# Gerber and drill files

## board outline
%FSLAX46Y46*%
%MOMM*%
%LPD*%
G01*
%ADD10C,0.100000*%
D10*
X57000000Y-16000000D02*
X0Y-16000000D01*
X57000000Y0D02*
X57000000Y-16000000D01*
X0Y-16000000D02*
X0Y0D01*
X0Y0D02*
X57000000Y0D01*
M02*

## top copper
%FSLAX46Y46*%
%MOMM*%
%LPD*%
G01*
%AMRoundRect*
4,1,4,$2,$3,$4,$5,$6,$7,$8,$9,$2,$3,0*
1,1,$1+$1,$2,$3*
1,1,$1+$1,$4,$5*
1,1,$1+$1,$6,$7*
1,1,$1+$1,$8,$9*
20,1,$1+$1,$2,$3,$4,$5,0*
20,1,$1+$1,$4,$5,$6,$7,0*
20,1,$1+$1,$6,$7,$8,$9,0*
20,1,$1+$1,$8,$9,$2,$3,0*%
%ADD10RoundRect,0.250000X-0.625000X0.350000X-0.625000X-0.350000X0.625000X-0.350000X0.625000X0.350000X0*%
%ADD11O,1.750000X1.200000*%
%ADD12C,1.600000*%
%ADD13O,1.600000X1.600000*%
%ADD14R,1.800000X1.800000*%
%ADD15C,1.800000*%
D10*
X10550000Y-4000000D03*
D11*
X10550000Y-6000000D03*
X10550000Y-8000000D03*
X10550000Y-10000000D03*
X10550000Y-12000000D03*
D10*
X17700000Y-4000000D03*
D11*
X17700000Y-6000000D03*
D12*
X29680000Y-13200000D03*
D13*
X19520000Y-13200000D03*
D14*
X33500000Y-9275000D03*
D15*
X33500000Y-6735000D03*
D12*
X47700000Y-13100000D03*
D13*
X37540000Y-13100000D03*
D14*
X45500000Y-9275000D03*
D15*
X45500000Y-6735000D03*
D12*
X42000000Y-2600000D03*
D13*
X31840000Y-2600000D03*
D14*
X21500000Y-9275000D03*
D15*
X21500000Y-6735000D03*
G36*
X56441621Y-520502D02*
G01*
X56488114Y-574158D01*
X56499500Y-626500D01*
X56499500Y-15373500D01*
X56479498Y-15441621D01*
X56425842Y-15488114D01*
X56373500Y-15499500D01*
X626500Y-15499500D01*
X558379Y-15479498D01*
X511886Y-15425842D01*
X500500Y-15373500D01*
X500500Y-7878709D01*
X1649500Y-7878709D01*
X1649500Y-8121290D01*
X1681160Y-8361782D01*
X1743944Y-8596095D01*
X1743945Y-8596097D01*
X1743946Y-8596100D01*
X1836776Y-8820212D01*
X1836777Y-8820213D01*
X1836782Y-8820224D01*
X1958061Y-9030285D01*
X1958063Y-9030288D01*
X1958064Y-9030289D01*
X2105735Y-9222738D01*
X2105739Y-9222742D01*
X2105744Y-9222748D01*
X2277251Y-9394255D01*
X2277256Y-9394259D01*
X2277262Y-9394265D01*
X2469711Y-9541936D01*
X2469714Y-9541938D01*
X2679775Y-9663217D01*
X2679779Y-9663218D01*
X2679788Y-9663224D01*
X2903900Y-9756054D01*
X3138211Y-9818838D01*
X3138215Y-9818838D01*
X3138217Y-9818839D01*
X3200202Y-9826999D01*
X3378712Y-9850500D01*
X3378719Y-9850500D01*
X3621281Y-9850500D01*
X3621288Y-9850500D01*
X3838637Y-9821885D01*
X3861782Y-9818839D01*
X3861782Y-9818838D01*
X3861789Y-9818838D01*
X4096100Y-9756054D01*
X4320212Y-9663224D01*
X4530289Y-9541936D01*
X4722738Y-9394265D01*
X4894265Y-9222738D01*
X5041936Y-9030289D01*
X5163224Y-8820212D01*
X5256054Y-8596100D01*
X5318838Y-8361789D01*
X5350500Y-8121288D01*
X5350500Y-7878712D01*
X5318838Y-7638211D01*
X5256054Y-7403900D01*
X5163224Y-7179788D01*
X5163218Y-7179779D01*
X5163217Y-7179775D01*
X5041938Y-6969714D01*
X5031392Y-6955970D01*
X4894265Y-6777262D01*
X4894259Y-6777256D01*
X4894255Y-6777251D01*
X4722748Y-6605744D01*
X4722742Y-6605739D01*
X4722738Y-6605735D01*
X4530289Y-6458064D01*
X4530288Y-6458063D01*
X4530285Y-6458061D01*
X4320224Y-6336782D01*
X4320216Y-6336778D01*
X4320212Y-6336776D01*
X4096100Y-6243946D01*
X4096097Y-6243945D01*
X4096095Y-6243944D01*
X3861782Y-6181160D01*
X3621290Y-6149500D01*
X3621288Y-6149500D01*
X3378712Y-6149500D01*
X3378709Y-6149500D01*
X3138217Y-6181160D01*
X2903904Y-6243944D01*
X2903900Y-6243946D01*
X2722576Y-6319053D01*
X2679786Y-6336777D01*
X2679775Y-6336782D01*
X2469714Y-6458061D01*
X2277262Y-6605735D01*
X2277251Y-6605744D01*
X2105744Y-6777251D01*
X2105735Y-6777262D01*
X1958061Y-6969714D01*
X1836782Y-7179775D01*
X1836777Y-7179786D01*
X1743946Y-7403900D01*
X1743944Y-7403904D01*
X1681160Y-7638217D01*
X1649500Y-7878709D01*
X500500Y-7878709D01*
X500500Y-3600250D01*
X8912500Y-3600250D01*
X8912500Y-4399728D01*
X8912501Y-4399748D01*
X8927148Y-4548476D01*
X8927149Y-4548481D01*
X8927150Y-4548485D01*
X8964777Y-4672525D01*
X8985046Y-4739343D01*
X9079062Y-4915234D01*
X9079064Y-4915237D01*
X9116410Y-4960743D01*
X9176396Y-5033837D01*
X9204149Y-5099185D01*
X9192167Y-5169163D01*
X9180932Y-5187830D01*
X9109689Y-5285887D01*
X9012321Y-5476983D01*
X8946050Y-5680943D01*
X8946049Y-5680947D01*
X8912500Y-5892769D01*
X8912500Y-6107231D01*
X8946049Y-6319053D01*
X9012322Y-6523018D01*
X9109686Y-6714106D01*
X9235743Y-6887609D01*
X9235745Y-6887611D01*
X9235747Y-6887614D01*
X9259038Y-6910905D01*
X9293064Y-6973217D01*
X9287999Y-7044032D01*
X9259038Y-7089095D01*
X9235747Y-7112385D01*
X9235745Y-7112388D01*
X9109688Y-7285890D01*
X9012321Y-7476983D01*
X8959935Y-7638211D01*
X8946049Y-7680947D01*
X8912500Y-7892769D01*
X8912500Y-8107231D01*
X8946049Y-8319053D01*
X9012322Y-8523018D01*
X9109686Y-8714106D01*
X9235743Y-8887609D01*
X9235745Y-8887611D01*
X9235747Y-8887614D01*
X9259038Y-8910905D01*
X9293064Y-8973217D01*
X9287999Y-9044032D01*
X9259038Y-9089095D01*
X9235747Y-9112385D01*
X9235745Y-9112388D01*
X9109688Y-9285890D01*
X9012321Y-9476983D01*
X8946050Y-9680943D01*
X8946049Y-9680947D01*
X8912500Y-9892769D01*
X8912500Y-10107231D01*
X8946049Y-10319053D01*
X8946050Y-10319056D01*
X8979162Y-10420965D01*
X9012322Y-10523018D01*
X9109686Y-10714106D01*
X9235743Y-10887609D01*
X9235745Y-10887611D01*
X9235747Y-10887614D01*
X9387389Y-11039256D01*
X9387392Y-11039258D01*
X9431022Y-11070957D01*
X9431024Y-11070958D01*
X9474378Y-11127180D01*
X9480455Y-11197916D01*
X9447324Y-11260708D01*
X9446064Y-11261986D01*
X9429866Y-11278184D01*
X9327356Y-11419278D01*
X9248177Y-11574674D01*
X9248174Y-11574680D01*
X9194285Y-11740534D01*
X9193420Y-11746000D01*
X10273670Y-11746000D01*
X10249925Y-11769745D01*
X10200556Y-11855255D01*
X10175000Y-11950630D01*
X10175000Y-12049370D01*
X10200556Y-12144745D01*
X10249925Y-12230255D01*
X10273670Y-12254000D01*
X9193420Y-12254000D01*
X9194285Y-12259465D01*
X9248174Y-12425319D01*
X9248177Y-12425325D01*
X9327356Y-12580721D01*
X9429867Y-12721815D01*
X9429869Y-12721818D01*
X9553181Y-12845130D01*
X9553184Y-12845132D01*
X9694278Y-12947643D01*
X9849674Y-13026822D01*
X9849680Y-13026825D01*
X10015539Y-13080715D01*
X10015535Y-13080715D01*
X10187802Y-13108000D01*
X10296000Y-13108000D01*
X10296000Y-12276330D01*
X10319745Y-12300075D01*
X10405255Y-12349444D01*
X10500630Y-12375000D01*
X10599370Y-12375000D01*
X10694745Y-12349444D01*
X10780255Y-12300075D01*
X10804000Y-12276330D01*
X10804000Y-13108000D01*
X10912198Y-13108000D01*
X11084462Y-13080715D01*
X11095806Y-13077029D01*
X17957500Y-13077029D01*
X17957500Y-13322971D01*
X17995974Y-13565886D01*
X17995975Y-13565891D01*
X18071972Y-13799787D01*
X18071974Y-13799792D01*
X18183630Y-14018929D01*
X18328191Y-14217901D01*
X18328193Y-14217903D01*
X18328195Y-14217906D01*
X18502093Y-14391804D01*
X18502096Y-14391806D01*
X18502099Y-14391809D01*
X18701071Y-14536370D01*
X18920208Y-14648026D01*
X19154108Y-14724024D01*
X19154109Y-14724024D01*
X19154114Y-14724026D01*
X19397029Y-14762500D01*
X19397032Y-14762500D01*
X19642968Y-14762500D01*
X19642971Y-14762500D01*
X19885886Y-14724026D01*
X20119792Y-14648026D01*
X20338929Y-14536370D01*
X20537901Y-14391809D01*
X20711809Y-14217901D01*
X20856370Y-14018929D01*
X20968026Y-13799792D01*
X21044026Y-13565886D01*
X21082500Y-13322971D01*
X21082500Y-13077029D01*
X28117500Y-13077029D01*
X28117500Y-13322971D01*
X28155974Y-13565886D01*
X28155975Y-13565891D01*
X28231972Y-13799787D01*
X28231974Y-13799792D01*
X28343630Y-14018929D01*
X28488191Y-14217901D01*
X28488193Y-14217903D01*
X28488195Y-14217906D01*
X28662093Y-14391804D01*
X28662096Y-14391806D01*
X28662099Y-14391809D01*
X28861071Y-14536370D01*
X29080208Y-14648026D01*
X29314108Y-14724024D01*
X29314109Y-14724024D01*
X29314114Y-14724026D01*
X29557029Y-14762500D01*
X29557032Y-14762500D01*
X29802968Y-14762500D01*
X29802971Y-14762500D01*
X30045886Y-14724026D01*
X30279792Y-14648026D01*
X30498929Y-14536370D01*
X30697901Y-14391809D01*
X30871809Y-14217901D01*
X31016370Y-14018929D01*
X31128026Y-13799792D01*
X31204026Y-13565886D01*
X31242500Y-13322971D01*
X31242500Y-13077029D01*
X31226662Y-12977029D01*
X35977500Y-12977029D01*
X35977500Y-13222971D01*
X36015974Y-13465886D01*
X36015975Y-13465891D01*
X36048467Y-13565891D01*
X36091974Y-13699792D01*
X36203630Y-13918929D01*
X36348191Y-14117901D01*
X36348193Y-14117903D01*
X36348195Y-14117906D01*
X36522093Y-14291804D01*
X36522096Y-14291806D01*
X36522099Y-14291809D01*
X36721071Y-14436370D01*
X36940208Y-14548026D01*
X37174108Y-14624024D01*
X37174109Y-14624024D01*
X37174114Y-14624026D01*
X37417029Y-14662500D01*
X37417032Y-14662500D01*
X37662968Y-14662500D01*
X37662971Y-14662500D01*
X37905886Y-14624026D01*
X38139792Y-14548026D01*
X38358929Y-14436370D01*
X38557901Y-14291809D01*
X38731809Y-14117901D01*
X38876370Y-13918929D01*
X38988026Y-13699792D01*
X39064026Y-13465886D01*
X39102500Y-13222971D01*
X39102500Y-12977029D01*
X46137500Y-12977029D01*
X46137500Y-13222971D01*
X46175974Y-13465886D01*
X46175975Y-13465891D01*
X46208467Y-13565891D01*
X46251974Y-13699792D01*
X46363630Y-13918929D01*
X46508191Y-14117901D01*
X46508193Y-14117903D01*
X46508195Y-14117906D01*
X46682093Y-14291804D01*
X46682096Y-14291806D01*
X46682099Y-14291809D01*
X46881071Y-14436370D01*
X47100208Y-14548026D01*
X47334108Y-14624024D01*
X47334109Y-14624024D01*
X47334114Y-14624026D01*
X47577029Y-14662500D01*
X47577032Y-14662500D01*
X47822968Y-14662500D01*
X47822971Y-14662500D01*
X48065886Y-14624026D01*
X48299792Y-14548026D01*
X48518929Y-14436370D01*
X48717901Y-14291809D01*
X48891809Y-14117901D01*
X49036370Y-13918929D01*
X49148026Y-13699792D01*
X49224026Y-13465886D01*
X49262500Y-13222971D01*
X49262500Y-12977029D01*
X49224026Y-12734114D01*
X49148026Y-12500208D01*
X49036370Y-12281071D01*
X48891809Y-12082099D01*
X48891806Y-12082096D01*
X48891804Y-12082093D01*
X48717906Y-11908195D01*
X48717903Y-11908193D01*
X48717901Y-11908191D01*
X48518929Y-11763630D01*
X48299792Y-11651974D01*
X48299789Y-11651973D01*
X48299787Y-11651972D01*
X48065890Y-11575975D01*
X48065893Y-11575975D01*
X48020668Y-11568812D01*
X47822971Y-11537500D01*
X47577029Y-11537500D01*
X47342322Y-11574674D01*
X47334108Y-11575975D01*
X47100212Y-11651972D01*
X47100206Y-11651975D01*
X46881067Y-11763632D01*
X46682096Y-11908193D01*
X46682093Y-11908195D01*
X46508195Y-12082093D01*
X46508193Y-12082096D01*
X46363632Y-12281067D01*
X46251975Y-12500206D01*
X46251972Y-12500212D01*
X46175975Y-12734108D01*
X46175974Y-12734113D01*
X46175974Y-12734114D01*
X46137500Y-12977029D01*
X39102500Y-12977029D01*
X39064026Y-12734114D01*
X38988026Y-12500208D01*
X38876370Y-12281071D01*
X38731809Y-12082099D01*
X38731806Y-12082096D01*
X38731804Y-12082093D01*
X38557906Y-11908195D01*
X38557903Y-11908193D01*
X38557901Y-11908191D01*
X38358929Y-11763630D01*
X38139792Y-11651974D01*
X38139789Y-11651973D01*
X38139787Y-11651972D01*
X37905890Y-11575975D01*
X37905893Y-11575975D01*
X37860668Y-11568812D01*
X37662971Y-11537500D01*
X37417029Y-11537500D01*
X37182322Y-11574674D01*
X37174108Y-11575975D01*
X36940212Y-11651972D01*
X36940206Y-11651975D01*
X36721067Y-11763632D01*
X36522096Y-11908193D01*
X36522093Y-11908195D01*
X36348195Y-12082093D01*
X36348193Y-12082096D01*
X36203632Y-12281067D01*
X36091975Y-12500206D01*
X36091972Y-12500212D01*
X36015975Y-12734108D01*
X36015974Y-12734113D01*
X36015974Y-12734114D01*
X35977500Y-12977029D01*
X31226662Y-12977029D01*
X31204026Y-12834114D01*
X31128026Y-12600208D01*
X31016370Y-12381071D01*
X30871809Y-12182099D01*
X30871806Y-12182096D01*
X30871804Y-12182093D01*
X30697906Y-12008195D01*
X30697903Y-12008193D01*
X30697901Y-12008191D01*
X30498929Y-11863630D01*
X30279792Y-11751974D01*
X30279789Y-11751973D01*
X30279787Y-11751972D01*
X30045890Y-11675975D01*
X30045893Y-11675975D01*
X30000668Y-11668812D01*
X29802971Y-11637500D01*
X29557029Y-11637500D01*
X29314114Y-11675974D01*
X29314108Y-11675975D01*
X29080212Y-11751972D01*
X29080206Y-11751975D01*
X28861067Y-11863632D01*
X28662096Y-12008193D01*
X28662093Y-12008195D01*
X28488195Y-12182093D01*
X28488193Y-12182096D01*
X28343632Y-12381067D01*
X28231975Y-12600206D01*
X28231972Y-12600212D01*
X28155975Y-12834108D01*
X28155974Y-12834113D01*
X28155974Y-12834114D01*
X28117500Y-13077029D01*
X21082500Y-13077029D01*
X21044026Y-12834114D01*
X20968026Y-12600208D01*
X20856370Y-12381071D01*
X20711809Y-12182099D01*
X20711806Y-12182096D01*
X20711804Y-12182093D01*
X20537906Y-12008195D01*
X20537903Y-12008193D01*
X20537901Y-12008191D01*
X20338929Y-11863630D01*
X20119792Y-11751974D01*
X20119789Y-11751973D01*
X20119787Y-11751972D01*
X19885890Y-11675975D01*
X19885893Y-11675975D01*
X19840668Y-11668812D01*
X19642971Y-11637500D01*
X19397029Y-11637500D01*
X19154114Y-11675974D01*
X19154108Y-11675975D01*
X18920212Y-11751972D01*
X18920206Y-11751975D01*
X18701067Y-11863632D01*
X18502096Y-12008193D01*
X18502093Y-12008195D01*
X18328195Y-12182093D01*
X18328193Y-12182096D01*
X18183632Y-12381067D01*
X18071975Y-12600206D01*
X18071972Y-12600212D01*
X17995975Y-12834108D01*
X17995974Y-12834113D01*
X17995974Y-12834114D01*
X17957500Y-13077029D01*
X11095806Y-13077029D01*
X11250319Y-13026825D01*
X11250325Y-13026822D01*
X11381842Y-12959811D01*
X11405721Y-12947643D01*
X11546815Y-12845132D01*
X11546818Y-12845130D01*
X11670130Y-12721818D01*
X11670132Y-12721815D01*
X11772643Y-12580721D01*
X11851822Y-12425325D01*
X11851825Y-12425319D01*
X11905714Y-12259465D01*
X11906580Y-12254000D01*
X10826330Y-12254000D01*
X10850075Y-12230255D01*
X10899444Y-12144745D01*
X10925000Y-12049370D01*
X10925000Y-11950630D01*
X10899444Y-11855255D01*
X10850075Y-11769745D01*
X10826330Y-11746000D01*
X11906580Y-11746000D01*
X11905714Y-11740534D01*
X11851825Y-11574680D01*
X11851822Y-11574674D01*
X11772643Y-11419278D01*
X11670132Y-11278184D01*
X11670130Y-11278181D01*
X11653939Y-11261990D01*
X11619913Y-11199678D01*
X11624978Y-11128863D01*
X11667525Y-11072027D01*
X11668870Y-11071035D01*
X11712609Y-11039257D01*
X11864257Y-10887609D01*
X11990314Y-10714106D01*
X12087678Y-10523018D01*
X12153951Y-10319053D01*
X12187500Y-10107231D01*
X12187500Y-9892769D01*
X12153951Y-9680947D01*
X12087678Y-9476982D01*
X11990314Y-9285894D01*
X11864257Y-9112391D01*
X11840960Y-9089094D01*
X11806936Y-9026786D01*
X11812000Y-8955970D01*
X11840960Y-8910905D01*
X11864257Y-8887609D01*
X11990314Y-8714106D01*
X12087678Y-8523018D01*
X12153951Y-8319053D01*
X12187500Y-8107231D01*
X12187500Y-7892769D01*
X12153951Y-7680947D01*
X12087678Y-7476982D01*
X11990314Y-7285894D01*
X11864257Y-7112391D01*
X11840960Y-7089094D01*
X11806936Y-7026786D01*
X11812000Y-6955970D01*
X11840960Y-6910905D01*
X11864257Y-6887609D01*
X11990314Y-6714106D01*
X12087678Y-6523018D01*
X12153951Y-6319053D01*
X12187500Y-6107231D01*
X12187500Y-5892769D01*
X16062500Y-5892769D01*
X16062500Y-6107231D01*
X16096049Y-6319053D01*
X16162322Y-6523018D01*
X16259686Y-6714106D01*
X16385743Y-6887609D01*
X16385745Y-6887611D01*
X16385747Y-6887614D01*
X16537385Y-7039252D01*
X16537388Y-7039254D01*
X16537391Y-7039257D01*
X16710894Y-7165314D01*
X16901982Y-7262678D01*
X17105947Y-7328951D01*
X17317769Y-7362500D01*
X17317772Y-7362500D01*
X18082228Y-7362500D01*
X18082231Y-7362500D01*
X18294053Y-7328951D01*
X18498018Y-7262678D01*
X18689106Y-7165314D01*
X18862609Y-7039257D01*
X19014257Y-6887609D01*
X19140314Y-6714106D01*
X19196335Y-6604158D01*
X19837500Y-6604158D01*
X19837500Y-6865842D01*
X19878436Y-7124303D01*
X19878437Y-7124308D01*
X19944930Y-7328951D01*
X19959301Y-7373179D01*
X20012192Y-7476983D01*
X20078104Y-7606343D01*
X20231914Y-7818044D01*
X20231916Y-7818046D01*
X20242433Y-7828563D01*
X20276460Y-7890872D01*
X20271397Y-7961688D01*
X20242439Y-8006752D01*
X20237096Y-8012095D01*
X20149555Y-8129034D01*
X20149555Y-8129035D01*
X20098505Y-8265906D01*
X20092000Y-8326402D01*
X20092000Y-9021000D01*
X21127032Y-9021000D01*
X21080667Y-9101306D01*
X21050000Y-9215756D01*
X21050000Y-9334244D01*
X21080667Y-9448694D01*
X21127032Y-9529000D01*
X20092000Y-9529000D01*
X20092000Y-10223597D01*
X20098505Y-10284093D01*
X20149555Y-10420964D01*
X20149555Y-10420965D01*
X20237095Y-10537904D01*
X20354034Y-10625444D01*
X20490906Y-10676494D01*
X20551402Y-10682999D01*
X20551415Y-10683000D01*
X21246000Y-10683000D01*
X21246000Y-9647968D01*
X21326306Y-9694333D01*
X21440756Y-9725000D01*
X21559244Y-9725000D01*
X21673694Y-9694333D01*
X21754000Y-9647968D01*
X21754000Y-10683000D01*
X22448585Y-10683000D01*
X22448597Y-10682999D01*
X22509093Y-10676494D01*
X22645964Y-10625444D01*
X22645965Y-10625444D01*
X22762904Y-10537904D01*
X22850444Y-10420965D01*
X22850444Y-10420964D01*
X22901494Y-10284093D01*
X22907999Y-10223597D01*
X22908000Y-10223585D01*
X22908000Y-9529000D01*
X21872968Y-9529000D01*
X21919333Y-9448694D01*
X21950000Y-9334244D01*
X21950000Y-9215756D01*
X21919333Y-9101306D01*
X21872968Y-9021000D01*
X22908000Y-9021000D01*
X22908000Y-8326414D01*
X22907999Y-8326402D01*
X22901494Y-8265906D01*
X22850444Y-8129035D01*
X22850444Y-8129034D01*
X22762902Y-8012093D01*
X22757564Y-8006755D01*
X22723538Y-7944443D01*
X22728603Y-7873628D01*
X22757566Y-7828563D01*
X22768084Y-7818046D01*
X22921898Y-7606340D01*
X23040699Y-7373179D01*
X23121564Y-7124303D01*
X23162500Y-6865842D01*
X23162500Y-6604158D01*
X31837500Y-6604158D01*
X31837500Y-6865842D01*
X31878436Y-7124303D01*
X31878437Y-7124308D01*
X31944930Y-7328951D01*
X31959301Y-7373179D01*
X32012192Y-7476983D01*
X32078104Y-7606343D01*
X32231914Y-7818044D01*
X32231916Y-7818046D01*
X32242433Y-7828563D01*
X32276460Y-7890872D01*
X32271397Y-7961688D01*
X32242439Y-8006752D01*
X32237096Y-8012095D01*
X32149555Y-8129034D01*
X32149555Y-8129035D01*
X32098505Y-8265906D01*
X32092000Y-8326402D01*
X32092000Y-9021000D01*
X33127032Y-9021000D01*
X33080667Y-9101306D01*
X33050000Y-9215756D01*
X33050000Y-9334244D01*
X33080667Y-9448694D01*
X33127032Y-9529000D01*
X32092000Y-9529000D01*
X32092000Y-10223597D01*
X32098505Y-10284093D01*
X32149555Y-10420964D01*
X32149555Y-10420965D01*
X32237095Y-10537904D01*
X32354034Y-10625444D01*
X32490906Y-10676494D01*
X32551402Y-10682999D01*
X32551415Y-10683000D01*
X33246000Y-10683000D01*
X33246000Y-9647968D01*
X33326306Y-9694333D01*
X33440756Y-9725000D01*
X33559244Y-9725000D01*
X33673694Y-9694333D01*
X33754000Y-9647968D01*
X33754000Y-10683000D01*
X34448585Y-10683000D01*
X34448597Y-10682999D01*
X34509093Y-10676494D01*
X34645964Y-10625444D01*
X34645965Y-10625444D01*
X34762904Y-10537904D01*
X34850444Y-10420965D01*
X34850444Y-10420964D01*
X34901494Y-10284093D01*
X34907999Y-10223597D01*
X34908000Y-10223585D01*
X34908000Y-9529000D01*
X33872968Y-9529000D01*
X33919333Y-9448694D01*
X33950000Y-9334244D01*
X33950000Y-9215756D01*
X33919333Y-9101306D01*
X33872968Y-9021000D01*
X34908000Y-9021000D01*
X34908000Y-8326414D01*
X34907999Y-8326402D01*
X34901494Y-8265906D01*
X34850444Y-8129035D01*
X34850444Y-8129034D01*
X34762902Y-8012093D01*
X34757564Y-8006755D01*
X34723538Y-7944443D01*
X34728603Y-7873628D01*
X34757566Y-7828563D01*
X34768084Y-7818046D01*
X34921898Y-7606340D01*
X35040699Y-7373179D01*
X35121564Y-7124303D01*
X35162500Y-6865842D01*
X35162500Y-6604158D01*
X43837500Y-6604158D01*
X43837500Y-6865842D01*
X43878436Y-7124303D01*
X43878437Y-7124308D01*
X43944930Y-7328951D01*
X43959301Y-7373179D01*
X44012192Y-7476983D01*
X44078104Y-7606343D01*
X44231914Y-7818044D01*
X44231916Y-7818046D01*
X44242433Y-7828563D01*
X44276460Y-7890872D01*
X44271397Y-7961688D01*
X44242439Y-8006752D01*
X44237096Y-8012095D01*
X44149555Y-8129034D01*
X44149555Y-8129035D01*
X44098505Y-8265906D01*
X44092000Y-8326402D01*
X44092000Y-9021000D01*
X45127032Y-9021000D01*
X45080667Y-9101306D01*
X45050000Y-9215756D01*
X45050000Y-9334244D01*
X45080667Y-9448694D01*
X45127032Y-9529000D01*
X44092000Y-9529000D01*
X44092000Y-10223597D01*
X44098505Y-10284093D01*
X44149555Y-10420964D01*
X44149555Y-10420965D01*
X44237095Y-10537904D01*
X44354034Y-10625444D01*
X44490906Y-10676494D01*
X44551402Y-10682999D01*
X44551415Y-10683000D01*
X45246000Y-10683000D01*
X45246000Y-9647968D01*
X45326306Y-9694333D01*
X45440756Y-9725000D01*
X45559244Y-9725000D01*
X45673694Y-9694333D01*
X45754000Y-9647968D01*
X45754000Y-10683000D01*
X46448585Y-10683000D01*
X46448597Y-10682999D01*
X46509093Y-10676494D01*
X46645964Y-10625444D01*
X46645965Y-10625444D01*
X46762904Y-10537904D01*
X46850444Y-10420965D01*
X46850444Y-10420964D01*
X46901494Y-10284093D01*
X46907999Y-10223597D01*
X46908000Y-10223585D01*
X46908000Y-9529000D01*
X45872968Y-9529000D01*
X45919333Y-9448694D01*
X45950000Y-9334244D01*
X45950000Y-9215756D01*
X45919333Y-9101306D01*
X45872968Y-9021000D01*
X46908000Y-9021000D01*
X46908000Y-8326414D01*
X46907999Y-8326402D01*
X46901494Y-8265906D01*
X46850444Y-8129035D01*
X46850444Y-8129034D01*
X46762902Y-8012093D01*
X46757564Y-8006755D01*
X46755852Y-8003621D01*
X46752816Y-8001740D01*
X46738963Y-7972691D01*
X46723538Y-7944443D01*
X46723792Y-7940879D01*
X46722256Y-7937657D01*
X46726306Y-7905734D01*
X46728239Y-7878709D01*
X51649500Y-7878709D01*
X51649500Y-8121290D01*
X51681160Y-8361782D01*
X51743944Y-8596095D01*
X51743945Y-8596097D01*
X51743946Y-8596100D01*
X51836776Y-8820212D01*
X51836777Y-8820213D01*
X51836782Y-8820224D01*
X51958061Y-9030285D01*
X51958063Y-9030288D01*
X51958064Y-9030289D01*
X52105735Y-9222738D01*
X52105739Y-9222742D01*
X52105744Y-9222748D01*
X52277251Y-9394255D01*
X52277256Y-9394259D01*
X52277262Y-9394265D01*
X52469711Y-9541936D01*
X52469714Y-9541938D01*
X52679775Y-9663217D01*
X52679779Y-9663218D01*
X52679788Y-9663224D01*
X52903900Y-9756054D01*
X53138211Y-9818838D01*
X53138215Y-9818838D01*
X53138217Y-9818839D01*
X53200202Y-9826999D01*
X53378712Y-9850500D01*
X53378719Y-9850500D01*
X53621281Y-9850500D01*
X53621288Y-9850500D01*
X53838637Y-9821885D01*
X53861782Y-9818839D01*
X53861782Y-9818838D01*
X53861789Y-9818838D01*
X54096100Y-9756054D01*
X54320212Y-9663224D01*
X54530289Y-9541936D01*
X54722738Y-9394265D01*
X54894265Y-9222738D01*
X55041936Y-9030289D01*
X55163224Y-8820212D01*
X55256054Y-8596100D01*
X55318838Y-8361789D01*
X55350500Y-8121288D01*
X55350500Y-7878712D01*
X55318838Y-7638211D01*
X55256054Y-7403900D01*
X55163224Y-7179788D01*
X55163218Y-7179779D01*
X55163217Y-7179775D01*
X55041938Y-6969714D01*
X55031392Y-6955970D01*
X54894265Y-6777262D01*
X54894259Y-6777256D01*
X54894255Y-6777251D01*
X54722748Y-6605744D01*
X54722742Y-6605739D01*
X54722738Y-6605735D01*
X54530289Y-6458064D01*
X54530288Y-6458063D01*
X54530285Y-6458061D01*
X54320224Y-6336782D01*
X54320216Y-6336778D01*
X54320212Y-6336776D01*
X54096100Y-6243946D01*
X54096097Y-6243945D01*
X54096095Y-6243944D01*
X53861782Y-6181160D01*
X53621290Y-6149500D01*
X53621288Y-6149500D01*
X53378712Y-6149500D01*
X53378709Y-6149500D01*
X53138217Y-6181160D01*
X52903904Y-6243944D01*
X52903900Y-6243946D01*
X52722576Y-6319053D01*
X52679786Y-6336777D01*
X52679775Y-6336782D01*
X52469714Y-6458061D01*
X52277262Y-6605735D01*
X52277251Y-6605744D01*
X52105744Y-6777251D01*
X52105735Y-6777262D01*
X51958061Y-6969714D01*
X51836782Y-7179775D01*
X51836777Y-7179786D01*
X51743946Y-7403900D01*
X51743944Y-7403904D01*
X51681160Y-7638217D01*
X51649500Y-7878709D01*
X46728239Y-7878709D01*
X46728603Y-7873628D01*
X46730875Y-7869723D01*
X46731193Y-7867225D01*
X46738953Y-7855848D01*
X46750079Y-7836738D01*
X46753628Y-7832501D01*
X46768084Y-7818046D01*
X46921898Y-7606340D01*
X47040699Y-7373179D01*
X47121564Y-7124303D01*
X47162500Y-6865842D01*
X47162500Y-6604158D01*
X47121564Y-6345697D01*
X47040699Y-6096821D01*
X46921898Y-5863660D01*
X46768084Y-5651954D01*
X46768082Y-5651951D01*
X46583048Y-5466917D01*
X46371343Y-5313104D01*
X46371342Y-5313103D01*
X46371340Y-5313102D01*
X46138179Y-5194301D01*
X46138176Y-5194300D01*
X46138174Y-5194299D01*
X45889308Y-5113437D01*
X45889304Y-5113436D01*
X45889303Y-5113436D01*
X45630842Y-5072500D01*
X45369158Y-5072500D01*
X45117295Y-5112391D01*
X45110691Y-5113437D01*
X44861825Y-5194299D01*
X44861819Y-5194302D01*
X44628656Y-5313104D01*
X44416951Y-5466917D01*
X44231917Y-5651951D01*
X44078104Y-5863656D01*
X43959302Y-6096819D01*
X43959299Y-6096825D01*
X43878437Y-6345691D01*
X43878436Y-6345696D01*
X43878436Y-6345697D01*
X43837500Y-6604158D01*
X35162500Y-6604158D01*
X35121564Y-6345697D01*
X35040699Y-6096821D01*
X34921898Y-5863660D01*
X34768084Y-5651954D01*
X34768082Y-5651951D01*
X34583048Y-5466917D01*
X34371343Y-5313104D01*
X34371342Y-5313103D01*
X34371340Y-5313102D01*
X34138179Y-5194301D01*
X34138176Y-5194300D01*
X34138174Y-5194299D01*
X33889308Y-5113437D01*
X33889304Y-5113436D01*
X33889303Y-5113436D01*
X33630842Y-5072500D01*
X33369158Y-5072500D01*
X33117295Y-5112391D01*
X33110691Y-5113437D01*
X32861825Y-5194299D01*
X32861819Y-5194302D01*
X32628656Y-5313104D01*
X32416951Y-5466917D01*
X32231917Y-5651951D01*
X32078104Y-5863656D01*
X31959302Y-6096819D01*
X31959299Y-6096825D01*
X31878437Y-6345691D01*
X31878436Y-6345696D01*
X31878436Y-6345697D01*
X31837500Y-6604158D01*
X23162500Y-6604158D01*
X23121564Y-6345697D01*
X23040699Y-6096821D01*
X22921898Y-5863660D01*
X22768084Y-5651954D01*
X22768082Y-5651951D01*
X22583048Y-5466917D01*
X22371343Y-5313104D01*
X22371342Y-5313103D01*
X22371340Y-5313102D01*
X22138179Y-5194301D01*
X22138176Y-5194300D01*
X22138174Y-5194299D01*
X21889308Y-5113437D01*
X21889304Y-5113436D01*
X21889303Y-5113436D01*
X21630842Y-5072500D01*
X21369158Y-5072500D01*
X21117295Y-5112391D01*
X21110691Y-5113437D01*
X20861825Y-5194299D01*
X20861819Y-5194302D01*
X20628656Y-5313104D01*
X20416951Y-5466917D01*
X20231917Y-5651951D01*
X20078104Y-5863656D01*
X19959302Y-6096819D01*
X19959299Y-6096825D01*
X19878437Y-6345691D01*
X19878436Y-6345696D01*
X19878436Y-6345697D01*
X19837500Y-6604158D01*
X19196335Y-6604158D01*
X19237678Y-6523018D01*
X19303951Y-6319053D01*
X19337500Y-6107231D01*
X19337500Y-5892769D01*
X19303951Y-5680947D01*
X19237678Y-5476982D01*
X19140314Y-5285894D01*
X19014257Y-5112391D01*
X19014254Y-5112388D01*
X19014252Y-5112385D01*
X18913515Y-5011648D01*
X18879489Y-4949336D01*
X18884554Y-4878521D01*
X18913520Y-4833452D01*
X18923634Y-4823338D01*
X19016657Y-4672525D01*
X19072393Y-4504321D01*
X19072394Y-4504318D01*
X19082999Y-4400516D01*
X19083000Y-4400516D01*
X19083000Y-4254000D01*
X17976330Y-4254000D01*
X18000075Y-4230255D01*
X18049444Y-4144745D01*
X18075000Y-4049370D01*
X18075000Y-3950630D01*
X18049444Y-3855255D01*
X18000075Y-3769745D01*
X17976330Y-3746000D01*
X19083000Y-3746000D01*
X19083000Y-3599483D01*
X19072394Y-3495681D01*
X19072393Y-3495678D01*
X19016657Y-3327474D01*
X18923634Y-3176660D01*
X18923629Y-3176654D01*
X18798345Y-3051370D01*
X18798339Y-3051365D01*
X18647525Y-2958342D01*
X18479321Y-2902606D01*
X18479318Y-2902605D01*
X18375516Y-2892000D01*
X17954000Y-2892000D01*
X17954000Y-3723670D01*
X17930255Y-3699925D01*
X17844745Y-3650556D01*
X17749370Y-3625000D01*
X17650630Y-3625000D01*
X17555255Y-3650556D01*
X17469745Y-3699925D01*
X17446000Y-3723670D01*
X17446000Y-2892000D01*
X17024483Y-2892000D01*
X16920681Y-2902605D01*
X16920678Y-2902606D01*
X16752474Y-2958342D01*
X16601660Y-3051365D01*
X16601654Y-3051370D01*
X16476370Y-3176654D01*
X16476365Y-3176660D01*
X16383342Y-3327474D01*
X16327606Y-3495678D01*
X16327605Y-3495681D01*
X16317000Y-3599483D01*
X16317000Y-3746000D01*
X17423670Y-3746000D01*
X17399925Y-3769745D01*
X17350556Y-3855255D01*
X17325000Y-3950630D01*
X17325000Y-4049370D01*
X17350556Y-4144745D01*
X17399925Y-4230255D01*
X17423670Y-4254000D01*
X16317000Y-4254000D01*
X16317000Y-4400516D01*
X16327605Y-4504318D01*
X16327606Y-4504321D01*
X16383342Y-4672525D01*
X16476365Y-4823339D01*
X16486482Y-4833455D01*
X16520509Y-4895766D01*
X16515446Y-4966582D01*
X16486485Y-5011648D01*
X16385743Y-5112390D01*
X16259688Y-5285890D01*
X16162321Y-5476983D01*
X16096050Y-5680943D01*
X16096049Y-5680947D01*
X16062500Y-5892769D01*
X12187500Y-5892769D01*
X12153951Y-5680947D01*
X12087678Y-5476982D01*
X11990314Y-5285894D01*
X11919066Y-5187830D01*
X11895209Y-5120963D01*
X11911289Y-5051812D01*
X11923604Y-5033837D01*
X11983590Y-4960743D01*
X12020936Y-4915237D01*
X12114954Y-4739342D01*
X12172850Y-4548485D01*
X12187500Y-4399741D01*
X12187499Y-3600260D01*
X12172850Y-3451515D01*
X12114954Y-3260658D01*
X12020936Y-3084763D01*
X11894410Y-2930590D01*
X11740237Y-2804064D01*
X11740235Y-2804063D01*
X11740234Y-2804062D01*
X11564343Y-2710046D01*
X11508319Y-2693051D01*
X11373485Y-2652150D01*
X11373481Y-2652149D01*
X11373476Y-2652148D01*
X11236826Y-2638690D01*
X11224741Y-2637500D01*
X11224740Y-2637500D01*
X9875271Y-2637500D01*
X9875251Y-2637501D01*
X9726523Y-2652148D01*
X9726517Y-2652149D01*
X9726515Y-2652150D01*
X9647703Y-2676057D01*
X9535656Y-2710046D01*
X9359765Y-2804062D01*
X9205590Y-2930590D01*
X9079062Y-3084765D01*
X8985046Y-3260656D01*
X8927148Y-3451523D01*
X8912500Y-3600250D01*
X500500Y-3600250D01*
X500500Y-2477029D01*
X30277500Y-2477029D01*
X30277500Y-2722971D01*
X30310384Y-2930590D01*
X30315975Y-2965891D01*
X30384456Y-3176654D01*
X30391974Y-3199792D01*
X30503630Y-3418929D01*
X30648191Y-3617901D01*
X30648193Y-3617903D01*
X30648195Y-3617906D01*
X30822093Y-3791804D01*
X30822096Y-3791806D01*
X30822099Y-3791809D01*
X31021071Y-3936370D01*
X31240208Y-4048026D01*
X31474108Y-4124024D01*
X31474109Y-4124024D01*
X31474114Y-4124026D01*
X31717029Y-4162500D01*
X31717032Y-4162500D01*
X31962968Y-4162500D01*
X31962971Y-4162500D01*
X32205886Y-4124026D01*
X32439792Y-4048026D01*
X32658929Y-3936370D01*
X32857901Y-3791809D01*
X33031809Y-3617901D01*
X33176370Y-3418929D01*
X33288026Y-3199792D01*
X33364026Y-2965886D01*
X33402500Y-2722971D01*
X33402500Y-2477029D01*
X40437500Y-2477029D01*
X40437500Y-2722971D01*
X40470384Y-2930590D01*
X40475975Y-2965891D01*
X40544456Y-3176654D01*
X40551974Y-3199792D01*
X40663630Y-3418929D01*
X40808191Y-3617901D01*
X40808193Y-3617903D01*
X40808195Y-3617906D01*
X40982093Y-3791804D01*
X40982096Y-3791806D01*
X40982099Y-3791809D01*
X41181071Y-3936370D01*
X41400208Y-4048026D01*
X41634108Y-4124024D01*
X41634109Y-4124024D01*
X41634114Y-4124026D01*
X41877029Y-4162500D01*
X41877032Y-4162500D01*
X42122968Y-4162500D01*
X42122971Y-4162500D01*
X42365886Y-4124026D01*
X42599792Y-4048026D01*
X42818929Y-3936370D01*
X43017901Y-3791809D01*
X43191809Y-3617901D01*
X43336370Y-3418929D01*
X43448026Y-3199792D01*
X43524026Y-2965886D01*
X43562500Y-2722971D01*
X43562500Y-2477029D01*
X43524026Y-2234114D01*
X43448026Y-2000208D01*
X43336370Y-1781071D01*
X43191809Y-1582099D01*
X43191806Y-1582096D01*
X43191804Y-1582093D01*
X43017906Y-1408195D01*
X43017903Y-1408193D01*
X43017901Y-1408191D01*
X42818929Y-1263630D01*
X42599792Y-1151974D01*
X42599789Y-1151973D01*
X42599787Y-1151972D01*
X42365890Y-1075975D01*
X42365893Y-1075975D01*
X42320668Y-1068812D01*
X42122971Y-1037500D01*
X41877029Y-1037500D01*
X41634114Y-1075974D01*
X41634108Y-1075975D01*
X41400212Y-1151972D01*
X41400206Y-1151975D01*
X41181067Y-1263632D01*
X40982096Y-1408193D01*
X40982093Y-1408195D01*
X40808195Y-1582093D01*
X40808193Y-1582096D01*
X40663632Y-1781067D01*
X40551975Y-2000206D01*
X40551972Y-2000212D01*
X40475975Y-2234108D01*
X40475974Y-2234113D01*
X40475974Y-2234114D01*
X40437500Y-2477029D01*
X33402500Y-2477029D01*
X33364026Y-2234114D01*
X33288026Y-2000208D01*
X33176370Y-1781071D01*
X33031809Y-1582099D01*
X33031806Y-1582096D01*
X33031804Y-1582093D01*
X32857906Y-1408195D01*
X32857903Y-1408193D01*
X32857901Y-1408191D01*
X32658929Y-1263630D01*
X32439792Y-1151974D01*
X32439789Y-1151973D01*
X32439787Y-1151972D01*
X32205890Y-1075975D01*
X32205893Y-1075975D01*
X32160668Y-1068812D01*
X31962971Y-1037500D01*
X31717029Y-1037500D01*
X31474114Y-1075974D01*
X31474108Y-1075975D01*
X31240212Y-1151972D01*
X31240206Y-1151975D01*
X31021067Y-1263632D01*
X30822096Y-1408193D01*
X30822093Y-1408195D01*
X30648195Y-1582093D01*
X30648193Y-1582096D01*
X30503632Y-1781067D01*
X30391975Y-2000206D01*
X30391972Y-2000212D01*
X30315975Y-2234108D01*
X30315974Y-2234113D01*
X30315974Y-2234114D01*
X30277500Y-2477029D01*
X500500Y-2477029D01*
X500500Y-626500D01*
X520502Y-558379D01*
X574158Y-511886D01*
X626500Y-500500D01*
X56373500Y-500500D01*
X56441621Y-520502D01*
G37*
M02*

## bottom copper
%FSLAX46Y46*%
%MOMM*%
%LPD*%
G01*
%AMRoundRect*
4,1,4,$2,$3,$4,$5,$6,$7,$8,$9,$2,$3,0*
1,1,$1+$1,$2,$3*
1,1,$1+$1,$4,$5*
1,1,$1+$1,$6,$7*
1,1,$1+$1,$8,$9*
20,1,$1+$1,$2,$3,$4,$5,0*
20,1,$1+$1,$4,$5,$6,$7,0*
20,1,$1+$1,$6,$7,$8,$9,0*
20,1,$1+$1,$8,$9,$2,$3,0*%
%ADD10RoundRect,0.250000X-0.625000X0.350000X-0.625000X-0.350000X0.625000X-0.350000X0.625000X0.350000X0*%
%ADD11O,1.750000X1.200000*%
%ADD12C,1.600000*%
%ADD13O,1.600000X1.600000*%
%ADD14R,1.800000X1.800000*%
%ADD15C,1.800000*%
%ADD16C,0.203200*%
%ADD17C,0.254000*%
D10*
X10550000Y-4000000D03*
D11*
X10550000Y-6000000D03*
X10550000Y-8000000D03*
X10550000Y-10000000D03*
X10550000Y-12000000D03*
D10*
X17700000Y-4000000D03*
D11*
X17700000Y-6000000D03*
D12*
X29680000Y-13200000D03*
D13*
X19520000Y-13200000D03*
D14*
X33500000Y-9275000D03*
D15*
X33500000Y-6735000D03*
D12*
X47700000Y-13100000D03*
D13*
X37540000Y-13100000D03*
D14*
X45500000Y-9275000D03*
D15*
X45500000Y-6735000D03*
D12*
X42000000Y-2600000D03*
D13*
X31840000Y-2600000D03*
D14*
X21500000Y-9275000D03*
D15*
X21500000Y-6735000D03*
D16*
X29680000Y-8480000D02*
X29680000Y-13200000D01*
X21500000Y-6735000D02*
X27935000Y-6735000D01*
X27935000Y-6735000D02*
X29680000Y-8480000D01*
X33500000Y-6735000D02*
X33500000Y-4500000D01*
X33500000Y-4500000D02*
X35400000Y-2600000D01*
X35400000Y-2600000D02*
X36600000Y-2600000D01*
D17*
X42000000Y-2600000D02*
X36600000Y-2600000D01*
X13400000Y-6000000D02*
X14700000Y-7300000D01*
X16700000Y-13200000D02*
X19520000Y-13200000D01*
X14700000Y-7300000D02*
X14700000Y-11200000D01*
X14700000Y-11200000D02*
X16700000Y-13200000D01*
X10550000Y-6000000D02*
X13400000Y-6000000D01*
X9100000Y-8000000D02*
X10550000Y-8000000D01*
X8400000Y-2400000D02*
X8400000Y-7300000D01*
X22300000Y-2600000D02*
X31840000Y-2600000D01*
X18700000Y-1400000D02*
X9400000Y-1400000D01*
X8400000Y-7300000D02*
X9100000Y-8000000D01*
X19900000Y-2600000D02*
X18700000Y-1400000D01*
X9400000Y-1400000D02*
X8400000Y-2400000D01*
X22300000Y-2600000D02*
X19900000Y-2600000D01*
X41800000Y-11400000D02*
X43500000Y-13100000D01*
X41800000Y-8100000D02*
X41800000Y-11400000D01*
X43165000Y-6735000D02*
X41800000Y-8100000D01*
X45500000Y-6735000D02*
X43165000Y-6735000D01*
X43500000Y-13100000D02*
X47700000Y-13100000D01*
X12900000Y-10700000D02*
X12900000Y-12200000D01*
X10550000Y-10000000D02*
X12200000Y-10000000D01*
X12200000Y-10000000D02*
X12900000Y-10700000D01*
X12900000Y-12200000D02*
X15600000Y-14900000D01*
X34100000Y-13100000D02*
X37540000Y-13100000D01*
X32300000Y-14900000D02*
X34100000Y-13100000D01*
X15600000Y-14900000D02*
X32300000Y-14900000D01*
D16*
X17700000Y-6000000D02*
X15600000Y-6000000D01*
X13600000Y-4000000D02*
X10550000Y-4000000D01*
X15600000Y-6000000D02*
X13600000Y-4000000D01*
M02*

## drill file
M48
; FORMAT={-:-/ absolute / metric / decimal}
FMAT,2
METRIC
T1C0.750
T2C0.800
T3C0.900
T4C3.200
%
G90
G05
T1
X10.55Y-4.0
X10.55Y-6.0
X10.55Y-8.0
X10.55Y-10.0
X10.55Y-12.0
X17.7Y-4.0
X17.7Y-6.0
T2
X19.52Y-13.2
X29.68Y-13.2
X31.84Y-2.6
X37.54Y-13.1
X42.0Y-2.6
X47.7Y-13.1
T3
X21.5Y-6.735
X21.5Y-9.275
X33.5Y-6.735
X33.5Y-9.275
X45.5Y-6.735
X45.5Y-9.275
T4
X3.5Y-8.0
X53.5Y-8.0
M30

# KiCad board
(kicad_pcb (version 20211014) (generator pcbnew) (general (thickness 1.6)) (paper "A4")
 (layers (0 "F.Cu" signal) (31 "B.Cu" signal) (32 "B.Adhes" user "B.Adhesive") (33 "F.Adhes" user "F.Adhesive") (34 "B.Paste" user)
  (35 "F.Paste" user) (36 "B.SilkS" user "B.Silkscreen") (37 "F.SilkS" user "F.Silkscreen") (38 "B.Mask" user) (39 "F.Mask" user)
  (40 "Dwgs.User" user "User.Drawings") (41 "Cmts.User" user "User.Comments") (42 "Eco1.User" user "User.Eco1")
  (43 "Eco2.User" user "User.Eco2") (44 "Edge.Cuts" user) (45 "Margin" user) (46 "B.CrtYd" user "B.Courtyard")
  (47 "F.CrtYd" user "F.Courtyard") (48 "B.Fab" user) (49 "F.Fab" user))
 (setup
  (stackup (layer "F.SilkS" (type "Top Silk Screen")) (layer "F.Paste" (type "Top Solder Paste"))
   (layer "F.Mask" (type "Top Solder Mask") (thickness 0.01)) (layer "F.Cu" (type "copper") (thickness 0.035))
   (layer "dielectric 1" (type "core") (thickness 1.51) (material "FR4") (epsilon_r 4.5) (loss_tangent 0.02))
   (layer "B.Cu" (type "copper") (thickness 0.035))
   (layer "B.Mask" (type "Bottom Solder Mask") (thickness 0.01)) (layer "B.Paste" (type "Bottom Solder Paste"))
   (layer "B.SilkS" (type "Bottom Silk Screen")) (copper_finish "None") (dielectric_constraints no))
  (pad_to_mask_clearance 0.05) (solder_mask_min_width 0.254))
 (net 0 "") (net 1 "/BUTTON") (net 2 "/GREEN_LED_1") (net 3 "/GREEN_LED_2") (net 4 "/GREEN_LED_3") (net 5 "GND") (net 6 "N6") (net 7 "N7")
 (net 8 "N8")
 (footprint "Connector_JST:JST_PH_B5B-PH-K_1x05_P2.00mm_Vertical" (layer "F.Cu") (at 10.55 4 -90)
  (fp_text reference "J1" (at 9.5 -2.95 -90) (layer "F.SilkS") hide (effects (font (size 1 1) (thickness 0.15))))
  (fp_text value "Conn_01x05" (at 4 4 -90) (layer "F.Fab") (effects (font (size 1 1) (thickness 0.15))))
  (pad "1" thru_hole roundrect (at 0 0 270) (size 1.2 1.75) (drill 0.75) (layers *.Cu *.Mask) (roundrect_rratio 0.2083333333)
   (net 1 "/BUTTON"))
  (pad "2" thru_hole oval (at 2 0 270) (size 1.2 1.75) (drill 0.75) (layers *.Cu *.Mask) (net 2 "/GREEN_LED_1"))
  (pad "3" thru_hole oval (at 4 0 270) (size 1.2 1.75) (drill 0.75) (layers *.Cu *.Mask) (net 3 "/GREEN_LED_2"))
  (pad "4" thru_hole oval (at 6 0 270) (size 1.2 1.75) (drill 0.75) (layers *.Cu *.Mask) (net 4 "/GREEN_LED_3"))
  (pad "5" thru_hole oval (at 8 0 270) (size 1.2 1.75) (drill 0.75) (layers *.Cu *.Mask) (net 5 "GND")))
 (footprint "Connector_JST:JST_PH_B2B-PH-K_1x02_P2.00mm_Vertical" (layer "F.Cu") (at 17.7 4 -90)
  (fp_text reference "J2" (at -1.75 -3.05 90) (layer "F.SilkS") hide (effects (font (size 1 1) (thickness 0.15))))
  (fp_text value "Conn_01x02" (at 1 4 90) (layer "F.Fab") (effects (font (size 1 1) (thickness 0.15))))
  (pad "1" thru_hole roundrect (at 0 0 270) (size 1.2 1.75) (drill 0.75) (layers *.Cu *.Mask) (roundrect_rratio 0.2083333333) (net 5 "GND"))
  (pad "2" thru_hole oval (at 2 0 270) (size 1.2 1.75) (drill 0.75) (layers *.Cu *.Mask) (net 1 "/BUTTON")))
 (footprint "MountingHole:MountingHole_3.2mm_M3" (layer "F.Cu") (at 53.5 8)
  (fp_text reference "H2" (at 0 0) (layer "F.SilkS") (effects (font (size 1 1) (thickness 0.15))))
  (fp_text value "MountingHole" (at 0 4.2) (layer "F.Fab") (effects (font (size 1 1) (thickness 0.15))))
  (pad "" np_thru_hole circle (at 0 0) (size 3.2 3.2) (drill 3.2) (layers *.Cu *.Mask)))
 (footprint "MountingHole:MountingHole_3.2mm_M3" (layer "F.Cu") (at 3.5 8)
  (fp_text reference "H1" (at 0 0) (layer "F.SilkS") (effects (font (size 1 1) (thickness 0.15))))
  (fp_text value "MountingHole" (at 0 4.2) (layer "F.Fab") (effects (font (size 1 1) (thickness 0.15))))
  (pad "" np_thru_hole circle (at 0 0) (size 3.2 3.2) (drill 3.2) (layers *.Cu *.Mask)))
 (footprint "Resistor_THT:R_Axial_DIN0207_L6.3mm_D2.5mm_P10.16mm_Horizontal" (layer "B.Cu") (at 29.68 13.2 180)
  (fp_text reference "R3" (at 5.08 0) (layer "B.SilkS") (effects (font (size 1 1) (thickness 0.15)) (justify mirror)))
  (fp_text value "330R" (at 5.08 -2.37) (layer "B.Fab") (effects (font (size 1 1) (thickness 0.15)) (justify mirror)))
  (pad "1" thru_hole circle (at 0 0 180) (size 1.6 1.6) (drill 0.8) (layers *.Cu *.Mask) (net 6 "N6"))
  (pad "2" thru_hole oval (at 10.16 0 180) (size 1.6 1.6) (drill 0.8) (layers *.Cu *.Mask) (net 2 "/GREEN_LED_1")))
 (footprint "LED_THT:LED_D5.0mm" (layer "B.Cu") (at 33.5 9.275 90)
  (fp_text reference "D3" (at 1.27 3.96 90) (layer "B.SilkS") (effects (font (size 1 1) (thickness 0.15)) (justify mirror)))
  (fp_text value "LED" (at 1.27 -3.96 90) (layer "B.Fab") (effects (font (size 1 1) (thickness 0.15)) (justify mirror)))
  (pad "1" thru_hole rect (at 0 0 90) (size 1.8 1.8) (drill 0.9) (layers *.Cu *.Mask) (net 5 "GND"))
  (pad "2" thru_hole circle (at 2.54 0 90) (size 1.8 1.8) (drill 0.9) (layers *.Cu *.Mask) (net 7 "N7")))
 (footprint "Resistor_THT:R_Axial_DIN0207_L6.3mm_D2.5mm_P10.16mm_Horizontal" (layer "B.Cu") (at 47.7 13.1 180)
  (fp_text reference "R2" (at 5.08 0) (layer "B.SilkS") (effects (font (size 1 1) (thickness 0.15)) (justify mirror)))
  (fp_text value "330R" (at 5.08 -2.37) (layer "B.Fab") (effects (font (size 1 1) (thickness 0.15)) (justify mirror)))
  (pad "1" thru_hole circle (at 0 0 180) (size 1.6 1.6) (drill 0.8) (layers *.Cu *.Mask) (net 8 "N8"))
  (pad "2" thru_hole oval (at 10.16 0 180) (size 1.6 1.6) (drill 0.8) (layers *.Cu *.Mask) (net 4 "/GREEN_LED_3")))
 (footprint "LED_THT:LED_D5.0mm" (layer "B.Cu") (at 45.5 9.275 90)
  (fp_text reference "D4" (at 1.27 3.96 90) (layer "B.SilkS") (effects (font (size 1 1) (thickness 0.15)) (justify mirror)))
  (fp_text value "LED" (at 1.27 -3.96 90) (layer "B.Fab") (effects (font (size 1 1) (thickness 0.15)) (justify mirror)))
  (pad "1" thru_hole rect (at 0 0 90) (size 1.8 1.8) (drill 0.9) (layers *.Cu *.Mask) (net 5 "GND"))
  (pad "2" thru_hole circle (at 2.54 0 90) (size 1.8 1.8) (drill 0.9) (layers *.Cu *.Mask) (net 8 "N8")))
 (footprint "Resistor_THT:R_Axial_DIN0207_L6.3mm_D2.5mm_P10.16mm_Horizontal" (layer "B.Cu") (at 42 2.6 180)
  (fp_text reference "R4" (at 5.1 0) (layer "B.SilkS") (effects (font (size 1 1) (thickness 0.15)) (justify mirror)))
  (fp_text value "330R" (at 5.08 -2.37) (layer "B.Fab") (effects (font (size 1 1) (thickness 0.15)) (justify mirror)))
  (pad "1" thru_hole circle (at 0 0 180) (size 1.6 1.6) (drill 0.8) (layers *.Cu *.Mask) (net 7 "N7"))
  (pad "2" thru_hole oval (at 10.16 0 180) (size 1.6 1.6) (drill 0.8) (layers *.Cu *.Mask) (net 3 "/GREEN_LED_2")))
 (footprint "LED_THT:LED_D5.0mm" (layer "B.Cu") (at 21.5 9.275 90)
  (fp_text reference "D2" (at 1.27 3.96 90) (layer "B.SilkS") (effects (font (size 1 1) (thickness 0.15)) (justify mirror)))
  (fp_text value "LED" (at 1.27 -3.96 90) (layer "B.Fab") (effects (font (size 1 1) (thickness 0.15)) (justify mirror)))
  (pad "1" thru_hole rect (at 0 0 90) (size 1.8 1.8) (drill 0.9) (layers *.Cu *.Mask) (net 5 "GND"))
  (pad "2" thru_hole circle (at 2.54 0 90) (size 1.8 1.8) (drill 0.9) (layers *.Cu *.Mask) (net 6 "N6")))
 (gr_line (start 57 16) (end 0 16) (layer "Edge.Cuts") (width 0.1))
 (gr_line (start 57 0) (end 57 16) (layer "Edge.Cuts") (width 0.1))
 (gr_line (start 0 16) (end 0 0) (layer "Edge.Cuts") (width 0.1))
 (gr_line (start 0 0) (end 57 0) (layer "Edge.Cuts") (width 0.1))
 (segment (start 29.68 8.48) (end 29.68 13.2) (width 0.2032) (layer "B.Cu") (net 6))
 (segment (start 21.5 6.735) (end 27.935 6.735) (width 0.2032) (layer "B.Cu") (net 6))
 (segment (start 27.935 6.735) (end 29.68 8.48) (width 0.2032) (layer "B.Cu") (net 6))
 (segment (start 33.5 6.735) (end 33.5 4.5) (width 0.2032) (layer "B.Cu") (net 7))
 (segment (start 33.5 4.5) (end 35.4 2.6) (width 0.2032) (layer "B.Cu") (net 7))
 (segment (start 35.4 2.6) (end 36.6 2.6) (width 0.2032) (layer "B.Cu") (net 7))
 (segment (start 42 2.6) (end 36.6 2.6) (width 0.254) (layer "B.Cu") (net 7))
 (segment (start 13.4 6) (end 14.7 7.3) (width 0.254) (layer "B.Cu") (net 2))
 (segment (start 16.7 13.2) (end 19.52 13.2) (width 0.254) (layer "B.Cu") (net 2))
 (segment (start 14.7 7.3) (end 14.7 11.2) (width 0.254) (layer "B.Cu") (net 2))
 (segment (start 14.7 11.2) (end 16.7 13.2) (width 0.254) (layer "B.Cu") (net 2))
 (segment (start 10.55 6) (end 13.4 6) (width 0.254) (layer "B.Cu") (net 2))
 (segment (start 9.1 8) (end 10.55 8) (width 0.254) (layer "B.Cu") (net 3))
 (segment (start 8.4 2.4) (end 8.4 7.3) (width 0.254) (layer "B.Cu") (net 3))
 (segment (start 22.3 2.6) (end 31.84 2.6) (width 0.254) (layer "B.Cu") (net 3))
 (segment (start 18.7 1.4) (end 9.4 1.4) (width 0.254) (layer "B.Cu") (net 3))
 (segment (start 8.4 7.3) (end 9.1 8) (width 0.254) (layer "B.Cu") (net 3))
 (segment (start 19.9 2.6) (end 18.7 1.4) (width 0.254) (layer "B.Cu") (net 3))
 (segment (start 9.4 1.4) (end 8.4 2.4) (width 0.254) (layer "B.Cu") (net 3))
 (segment (start 22.3 2.6) (end 19.9 2.6) (width 0.254) (layer "B.Cu") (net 3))
 (segment (start 41.8 11.4) (end 43.5 13.1) (width 0.254) (layer "B.Cu") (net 8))
 (segment (start 41.8 8.1) (end 41.8 11.4) (width 0.254) (layer "B.Cu") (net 8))
 (segment (start 43.165 6.735) (end 41.8 8.1) (width 0.254) (layer "B.Cu") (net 8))
 (segment (start 45.5 6.735) (end 43.165 6.735) (width 0.254) (layer "B.Cu") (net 8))
 (segment (start 43.5 13.1) (end 47.7 13.1) (width 0.254) (layer "B.Cu") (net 8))
 (segment (start 12.9 10.7) (end 12.9 12.2) (width 0.254) (layer "B.Cu") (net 4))
 (segment (start 10.55 10) (end 12.2 10) (width 0.254) (layer "B.Cu") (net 4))
 (segment (start 12.2 10) (end 12.9 10.7) (width 0.254) (layer "B.Cu") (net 4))
 (segment (start 12.9 12.2) (end 15.6 14.9) (width 0.254) (layer "B.Cu") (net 4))
 (segment (start 34.1 13.1) (end 37.54 13.1) (width 0.254) (layer "B.Cu") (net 4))
 (segment (start 32.3 14.9) (end 34.1 13.1) (width 0.254) (layer "B.Cu") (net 4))
 (segment (start 15.6 14.9) (end 32.3 14.9) (width 0.254) (layer "B.Cu") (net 4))
 (segment (start 17.7 6) (end 15.6 6) (width 0.2032) (layer "B.Cu") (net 1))
 (segment (start 13.6 4) (end 10.55 4) (width 0.2032) (layer "B.Cu") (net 1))
 (segment (start 15.6 6) (end 13.6 4) (width 0.2032) (layer "B.Cu") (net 1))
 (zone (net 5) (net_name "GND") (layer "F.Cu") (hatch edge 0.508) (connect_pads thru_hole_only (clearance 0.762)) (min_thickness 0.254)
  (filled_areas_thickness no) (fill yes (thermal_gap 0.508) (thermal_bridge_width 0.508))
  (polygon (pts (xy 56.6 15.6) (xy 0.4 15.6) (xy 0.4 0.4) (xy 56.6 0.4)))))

